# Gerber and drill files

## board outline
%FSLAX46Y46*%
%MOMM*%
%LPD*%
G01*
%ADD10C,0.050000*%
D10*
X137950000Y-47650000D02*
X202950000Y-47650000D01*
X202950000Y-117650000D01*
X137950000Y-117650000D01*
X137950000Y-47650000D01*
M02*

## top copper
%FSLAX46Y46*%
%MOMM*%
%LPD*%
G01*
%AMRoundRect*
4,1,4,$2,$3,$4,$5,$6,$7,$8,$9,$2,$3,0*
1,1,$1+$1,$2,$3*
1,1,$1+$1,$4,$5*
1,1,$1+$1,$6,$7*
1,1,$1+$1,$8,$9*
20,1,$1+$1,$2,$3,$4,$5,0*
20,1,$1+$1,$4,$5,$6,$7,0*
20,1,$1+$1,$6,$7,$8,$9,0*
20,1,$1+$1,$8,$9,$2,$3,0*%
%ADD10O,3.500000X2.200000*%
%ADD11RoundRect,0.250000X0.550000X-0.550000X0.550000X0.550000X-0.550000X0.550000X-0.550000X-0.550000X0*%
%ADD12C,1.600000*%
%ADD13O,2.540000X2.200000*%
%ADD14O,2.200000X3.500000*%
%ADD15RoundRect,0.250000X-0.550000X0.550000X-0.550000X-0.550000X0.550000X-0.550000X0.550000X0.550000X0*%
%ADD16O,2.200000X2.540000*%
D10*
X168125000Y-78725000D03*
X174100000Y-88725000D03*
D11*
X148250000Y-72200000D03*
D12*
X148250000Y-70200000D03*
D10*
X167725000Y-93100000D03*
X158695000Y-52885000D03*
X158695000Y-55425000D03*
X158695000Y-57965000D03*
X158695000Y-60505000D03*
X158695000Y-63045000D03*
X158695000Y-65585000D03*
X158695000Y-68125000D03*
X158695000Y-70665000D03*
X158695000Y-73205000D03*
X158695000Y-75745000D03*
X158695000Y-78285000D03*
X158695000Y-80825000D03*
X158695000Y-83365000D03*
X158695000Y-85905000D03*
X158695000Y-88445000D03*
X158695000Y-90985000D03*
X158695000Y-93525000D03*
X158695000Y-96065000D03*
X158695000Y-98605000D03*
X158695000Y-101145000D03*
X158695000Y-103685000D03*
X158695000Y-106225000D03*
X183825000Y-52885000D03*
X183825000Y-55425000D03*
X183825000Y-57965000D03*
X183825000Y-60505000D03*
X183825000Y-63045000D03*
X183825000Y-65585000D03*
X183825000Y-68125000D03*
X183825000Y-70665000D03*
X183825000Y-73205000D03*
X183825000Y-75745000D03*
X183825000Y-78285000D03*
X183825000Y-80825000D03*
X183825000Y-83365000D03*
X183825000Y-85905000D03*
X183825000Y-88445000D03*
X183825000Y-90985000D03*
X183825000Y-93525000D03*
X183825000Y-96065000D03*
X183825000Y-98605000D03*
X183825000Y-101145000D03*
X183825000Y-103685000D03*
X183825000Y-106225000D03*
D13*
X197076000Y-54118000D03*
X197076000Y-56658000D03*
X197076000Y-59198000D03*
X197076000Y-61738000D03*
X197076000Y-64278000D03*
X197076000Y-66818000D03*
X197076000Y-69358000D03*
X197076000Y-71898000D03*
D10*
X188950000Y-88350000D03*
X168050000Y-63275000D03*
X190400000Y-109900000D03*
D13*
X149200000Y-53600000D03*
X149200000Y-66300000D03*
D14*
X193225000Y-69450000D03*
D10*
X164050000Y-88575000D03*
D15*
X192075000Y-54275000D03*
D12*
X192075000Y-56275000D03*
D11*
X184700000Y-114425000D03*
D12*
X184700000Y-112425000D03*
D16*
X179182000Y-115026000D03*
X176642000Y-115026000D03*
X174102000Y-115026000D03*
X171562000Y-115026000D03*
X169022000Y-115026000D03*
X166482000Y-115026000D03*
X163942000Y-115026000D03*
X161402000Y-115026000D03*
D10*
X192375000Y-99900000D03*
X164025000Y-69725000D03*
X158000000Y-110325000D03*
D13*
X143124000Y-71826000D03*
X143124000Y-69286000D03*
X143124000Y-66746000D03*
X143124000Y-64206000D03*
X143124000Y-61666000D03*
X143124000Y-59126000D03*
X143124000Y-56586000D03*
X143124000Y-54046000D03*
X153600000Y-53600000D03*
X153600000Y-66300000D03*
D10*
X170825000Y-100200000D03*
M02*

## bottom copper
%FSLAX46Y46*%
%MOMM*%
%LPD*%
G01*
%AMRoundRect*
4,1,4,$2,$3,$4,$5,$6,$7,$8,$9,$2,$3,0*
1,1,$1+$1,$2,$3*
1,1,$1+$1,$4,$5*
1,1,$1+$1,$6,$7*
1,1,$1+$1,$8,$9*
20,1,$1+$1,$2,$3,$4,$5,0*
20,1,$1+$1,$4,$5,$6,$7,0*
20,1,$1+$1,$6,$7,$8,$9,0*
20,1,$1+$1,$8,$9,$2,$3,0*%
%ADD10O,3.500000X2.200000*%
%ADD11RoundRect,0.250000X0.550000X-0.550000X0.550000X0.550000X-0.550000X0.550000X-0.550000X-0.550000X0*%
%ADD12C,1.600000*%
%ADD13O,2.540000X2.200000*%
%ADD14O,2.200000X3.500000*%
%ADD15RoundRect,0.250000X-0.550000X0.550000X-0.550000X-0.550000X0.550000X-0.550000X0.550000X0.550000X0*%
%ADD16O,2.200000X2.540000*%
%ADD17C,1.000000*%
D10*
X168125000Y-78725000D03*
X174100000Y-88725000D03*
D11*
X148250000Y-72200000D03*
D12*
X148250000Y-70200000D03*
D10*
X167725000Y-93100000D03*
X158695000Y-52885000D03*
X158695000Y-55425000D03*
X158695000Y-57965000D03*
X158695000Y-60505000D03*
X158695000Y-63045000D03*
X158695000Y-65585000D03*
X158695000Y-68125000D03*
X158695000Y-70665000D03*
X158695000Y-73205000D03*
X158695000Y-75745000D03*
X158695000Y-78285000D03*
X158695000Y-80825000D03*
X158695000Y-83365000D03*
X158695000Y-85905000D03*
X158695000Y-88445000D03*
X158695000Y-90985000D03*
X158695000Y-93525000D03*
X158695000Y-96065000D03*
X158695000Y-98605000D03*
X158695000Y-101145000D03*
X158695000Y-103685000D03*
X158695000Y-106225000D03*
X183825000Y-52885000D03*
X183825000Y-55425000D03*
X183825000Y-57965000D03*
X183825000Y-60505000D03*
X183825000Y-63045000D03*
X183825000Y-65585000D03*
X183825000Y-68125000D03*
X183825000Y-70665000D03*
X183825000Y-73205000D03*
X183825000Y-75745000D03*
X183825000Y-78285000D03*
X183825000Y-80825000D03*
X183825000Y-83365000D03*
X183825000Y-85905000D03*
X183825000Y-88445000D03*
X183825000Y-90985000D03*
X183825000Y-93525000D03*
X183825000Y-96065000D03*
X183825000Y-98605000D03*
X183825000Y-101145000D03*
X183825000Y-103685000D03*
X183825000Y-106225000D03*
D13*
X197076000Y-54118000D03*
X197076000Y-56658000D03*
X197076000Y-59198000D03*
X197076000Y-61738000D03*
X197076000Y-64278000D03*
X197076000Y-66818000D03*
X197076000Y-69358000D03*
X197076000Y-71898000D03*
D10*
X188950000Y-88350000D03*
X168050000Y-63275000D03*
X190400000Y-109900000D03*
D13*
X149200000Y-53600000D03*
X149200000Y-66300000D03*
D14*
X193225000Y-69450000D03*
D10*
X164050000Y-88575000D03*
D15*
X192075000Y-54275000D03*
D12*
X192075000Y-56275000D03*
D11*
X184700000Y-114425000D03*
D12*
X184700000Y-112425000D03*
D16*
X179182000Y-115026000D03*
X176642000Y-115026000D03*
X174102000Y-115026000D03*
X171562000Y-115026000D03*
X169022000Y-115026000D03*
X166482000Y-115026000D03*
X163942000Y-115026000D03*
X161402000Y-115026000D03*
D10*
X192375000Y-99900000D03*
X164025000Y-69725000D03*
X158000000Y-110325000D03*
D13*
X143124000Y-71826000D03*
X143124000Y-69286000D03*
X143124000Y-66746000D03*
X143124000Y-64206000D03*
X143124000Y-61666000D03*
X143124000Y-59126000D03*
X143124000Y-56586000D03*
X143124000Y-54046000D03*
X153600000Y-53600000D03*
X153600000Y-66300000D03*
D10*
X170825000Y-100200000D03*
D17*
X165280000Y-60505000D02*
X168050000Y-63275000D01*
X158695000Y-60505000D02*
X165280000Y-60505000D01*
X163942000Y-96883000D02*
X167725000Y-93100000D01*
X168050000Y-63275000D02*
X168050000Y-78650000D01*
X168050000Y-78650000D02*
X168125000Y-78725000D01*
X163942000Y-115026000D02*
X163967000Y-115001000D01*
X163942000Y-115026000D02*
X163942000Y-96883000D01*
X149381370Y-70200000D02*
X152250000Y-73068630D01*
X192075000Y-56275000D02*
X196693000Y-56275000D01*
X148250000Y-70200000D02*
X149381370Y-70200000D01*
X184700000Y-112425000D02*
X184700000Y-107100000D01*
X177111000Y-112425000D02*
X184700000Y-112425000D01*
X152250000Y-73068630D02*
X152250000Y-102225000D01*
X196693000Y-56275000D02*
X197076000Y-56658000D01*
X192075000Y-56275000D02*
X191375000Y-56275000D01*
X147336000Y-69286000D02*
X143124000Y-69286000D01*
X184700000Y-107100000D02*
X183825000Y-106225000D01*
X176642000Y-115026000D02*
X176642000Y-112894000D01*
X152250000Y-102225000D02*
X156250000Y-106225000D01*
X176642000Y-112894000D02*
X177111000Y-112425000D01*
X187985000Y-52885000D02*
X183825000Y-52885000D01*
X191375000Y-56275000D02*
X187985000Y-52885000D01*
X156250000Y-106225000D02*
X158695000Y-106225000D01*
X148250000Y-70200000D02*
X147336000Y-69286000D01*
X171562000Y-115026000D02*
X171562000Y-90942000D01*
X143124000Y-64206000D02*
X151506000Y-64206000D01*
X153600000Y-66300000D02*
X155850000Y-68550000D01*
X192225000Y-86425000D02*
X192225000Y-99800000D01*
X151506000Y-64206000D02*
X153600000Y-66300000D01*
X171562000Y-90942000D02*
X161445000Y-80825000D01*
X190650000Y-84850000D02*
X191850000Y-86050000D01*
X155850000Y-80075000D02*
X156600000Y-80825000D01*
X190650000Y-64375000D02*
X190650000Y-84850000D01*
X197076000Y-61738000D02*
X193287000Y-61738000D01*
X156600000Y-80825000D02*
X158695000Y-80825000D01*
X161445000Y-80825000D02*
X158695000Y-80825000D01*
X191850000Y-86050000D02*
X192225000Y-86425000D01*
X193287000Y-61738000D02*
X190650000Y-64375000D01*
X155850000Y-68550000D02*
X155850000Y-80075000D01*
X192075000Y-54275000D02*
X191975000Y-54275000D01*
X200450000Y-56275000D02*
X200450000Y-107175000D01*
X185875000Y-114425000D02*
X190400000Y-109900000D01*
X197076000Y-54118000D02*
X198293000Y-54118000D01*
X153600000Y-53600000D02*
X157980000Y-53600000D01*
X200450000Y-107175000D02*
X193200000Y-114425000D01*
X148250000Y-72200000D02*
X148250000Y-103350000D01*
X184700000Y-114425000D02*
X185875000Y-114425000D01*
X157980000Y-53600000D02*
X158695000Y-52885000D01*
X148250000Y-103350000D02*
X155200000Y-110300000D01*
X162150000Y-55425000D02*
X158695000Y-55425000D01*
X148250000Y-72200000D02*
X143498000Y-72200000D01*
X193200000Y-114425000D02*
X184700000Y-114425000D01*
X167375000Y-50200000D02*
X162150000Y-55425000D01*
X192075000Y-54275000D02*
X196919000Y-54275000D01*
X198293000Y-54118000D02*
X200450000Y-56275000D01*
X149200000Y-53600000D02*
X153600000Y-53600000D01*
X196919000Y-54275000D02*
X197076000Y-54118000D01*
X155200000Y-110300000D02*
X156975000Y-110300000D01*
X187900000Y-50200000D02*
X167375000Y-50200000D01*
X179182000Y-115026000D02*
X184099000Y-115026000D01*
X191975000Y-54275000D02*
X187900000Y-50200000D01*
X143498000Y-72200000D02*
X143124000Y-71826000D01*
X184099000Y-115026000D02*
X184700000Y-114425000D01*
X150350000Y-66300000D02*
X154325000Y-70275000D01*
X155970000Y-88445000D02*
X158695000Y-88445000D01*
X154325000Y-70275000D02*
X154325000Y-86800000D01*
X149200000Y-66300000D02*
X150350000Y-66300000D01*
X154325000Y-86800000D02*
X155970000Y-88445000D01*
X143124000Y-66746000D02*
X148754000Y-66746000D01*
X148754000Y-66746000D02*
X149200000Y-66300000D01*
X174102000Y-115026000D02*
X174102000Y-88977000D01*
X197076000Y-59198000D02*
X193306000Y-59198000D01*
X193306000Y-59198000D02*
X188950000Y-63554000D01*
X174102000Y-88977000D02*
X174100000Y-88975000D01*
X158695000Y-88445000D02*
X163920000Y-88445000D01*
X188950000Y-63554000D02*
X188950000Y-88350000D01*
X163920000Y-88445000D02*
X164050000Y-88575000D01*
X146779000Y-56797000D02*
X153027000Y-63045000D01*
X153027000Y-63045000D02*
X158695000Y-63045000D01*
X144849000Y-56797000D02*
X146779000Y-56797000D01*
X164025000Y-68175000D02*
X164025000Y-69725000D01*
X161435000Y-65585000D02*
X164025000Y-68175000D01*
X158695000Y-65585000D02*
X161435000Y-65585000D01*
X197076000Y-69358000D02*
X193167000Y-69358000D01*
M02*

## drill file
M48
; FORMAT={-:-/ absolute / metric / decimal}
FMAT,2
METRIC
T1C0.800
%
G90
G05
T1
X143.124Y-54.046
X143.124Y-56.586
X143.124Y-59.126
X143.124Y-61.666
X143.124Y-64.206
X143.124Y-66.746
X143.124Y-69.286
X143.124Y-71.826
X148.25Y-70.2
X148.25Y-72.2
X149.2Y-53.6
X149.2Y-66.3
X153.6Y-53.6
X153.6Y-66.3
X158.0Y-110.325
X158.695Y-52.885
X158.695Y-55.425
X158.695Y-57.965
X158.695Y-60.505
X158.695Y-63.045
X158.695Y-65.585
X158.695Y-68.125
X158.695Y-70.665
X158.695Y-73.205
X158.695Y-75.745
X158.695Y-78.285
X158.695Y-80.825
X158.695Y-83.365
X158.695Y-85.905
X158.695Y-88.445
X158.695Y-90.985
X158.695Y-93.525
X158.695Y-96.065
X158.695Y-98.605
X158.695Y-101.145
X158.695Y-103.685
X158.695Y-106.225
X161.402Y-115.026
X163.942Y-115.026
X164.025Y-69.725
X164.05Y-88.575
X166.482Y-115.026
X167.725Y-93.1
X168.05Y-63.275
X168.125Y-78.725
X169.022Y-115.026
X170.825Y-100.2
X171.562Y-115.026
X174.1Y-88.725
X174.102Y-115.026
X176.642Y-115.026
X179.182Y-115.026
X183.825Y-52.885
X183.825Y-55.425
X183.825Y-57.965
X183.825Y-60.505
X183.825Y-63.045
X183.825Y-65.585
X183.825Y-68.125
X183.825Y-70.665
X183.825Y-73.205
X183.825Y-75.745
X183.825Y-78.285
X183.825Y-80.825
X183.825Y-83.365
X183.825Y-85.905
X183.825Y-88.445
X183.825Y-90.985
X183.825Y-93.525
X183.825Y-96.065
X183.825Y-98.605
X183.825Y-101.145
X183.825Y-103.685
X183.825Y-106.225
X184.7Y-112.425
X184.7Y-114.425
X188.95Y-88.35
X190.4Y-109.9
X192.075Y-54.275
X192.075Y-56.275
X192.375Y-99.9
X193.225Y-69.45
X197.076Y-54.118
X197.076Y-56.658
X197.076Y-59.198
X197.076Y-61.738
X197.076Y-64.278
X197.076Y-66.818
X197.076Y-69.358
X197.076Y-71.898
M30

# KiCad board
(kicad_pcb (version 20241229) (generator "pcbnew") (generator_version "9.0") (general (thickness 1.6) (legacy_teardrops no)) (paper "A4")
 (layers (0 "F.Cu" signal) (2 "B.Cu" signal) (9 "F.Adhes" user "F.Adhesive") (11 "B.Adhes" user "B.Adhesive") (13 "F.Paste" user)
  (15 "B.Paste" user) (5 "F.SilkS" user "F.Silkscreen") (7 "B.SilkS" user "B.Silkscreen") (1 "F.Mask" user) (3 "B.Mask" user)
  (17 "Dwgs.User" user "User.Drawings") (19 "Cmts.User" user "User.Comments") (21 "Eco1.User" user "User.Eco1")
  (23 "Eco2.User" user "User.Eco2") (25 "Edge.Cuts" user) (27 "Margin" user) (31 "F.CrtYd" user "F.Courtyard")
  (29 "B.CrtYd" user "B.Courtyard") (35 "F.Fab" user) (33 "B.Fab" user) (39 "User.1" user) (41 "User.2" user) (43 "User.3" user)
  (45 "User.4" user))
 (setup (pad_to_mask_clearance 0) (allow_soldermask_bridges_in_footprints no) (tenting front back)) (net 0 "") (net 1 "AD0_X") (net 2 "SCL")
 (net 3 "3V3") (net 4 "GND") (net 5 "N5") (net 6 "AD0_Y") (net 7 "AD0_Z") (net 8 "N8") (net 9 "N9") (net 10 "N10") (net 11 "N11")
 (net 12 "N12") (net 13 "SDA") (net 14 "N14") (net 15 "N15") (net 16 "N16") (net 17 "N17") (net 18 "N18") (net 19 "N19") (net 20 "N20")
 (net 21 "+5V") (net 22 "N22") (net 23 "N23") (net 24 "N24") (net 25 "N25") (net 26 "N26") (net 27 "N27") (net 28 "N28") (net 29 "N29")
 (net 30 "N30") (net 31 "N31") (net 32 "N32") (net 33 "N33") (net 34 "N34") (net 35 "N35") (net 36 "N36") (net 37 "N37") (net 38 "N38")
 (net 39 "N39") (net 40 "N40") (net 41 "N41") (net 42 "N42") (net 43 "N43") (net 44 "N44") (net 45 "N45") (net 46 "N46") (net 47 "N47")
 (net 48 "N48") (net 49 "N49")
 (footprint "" (layer "F.Cu") (at 168.125 78.725)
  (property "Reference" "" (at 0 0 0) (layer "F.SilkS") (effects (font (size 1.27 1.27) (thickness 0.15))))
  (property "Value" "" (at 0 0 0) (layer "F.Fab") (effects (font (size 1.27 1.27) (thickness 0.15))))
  (pad "4" thru_hole oval (at 0 0) (size 3.5 2.2) (drill 0.8) (layers "*.Cu" "*.Mask") (remove_unused_layers no) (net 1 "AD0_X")))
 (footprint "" (layer "F.Cu") (at 174.1 88.725)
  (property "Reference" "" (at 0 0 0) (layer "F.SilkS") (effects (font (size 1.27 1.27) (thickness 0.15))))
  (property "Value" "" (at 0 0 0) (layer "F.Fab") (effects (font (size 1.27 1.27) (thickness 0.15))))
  (pad "SCL" thru_hole oval (at 0 0) (size 3.5 2.2) (drill 0.8) (layers "*.Cu" "*.Mask") (remove_unused_layers no) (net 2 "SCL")))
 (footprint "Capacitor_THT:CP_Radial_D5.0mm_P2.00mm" (layer "F.Cu") (at 148.25 72.2 90)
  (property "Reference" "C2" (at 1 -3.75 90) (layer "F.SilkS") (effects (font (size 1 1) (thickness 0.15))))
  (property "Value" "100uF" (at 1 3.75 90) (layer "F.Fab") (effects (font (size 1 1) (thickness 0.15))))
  (pad "1" thru_hole roundrect (at 0 0 90) (size 1.6 1.6) (drill 0.8) (layers "*.Cu" "*.Mask") (remove_unused_layers no)
   (roundrect_rratio 0.15625) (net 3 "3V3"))
  (pad "2" thru_hole circle (at 2 0 90) (size 1.6 1.6) (drill 0.8) (layers "*.Cu" "*.Mask") (remove_unused_layers no) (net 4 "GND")))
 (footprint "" (layer "F.Cu") (at 167.725 93.1)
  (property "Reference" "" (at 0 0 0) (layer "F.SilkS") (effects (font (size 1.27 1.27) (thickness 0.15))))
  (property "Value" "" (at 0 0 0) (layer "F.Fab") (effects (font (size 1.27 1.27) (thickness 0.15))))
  (pad "4" thru_hole oval (at 0 0) (size 3.5 2.2) (drill 0.8) (layers "*.Cu" "*.Mask") (remove_unused_layers no) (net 1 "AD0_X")))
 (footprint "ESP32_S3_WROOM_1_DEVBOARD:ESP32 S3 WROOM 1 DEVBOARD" (layer "F.Cu") (at 156.325 51.225)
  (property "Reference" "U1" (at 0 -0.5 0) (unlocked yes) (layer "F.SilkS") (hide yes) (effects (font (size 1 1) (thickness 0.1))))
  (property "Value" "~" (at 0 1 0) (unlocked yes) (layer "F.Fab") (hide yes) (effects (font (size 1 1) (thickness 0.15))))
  (pad "1" thru_hole oval (at 2.37 1.66) (size 3.5 2.2) (drill 0.8) (layers "*.Cu" "*.Mask") (remove_unused_layers no) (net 3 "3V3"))
  (pad "2" thru_hole oval (at 2.37 4.2) (size 3.5 2.2) (drill 0.8) (layers "*.Cu" "*.Mask") (remove_unused_layers no) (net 3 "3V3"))
  (pad "3" thru_hole oval (at 2.37 6.74) (size 3.5 2.2) (drill 0.8) (layers "*.Cu" "*.Mask") (remove_unused_layers no) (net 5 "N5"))
  (pad "4" thru_hole oval (at 2.37 9.28) (size 3.5 2.2) (drill 0.8) (layers "*.Cu" "*.Mask") (remove_unused_layers no) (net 1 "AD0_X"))
  (pad "5" thru_hole oval (at 2.37 11.82) (size 3.5 2.2) (drill 0.8) (layers "*.Cu" "*.Mask") (remove_unused_layers no) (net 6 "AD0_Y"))
  (pad "6" thru_hole oval (at 2.37 14.36) (size 3.5 2.2) (drill 0.8) (layers "*.Cu" "*.Mask") (remove_unused_layers no) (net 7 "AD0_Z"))
  (pad "7" thru_hole oval (at 2.37 16.9) (size 3.5 2.2) (drill 0.8) (layers "*.Cu" "*.Mask") (remove_unused_layers no) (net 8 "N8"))
  (pad "8" thru_hole oval (at 2.37 19.44) (size 3.5 2.2) (drill 0.8) (layers "*.Cu" "*.Mask") (remove_unused_layers no) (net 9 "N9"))
  (pad "9" thru_hole oval (at 2.37 21.98) (size 3.5 2.2) (drill 0.8) (layers "*.Cu" "*.Mask") (remove_unused_layers no) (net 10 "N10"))
  (pad "10" thru_hole oval (at 2.37 24.52) (size 3.5 2.2) (drill 0.8) (layers "*.Cu" "*.Mask") (remove_unused_layers no) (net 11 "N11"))
  (pad "11" thru_hole oval (at 2.37 27.06) (size 3.5 2.2) (drill 0.8) (layers "*.Cu" "*.Mask") (remove_unused_layers no) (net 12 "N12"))
  (pad "12" thru_hole oval (at 2.37 29.6) (size 3.5 2.2) (drill 0.8) (layers "*.Cu" "*.Mask") (remove_unused_layers no) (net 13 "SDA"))
  (pad "13" thru_hole oval (at 2.37 32.14) (size 3.5 2.2) (drill 0.8) (layers "*.Cu" "*.Mask") (remove_unused_layers no) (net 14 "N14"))
  (pad "14" thru_hole oval (at 2.37 34.68) (size 3.5 2.2) (drill 0.8) (layers "*.Cu" "*.Mask") (remove_unused_layers no) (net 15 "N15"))
  (pad "15" thru_hole oval (at 2.37 37.22) (size 3.5 2.2) (drill 0.8) (layers "*.Cu" "*.Mask") (remove_unused_layers no) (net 2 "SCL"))
  (pad "16" thru_hole oval (at 2.37 39.76) (size 3.5 2.2) (drill 0.8) (layers "*.Cu" "*.Mask") (remove_unused_layers no) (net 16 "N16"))
  (pad "17" thru_hole oval (at 2.37 42.3) (size 3.5 2.2) (drill 0.8) (layers "*.Cu" "*.Mask") (remove_unused_layers no) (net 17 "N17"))
  (pad "18" thru_hole oval (at 2.37 44.84) (size 3.5 2.2) (drill 0.8) (layers "*.Cu" "*.Mask") (remove_unused_layers no) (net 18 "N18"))
  (pad "19" thru_hole oval (at 2.37 47.38) (size 3.5 2.2) (drill 0.8) (layers "*.Cu" "*.Mask") (remove_unused_layers no) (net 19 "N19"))
  (pad "20" thru_hole oval (at 2.37 49.92) (size 3.5 2.2) (drill 0.8) (layers "*.Cu" "*.Mask") (remove_unused_layers no) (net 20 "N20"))
  (pad "21" thru_hole oval (at 2.37 52.46) (size 3.5 2.2) (drill 0.8) (layers "*.Cu" "*.Mask") (remove_unused_layers no) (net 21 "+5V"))
  (pad "22" thru_hole oval (at 2.37 55) (size 3.5 2.2) (drill 0.8) (layers "*.Cu" "*.Mask") (remove_unused_layers no) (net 4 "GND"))
  (pad "23" thru_hole oval (at 27.5 1.66) (size 3.5 2.2) (drill 0.8) (layers "*.Cu" "*.Mask") (remove_unused_layers no) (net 4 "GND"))
  (pad "24" thru_hole oval (at 27.5 4.2) (size 3.5 2.2) (drill 0.8) (layers "*.Cu" "*.Mask") (remove_unused_layers no) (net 4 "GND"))
  (pad "25" thru_hole oval (at 27.5 6.74) (size 3.5 2.2) (drill 0.8) (layers "*.Cu" "*.Mask") (remove_unused_layers no) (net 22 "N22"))
  (pad "26" thru_hole oval (at 27.5 9.28) (size 3.5 2.2) (drill 0.8) (layers "*.Cu" "*.Mask") (remove_unused_layers no) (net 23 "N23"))
  (pad "27" thru_hole oval (at 27.5 11.82) (size 3.5 2.2) (drill 0.8) (layers "*.Cu" "*.Mask") (remove_unused_layers no) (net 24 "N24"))
  (pad "28" thru_hole oval (at 27.5 14.36) (size 3.5 2.2) (drill 0.8) (layers "*.Cu" "*.Mask") (remove_unused_layers no) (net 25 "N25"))
  (pad "29" thru_hole oval (at 27.5 16.9) (size 3.5 2.2) (drill 0.8) (layers "*.Cu" "*.Mask") (remove_unused_layers no) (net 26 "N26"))
  (pad "30" thru_hole oval (at 27.5 19.44) (size 3.5 2.2) (drill 0.8) (layers "*.Cu" "*.Mask") (remove_unused_layers no) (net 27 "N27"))
  (pad "31" thru_hole oval (at 27.5 21.98) (size 3.5 2.2) (drill 0.8) (layers "*.Cu" "*.Mask") (remove_unused_layers no) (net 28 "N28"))
  (pad "32" thru_hole oval (at 27.5 24.52) (size 3.5 2.2) (drill 0.8) (layers "*.Cu" "*.Mask") (remove_unused_layers no) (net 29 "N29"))
  (pad "33" thru_hole oval (at 27.5 27.06) (size 3.5 2.2) (drill 0.8) (layers "*.Cu" "*.Mask") (remove_unused_layers no) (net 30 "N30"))
  (pad "34" thru_hole oval (at 27.5 29.6) (size 3.5 2.2) (drill 0.8) (layers "*.Cu" "*.Mask") (remove_unused_layers no) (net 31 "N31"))
  (pad "35" thru_hole oval (at 27.5 32.14) (size 3.5 2.2) (drill 0.8) (layers "*.Cu" "*.Mask") (remove_unused_layers no) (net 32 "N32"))
  (pad "36" thru_hole oval (at 27.5 34.68) (size 3.5 2.2) (drill 0.8) (layers "*.Cu" "*.Mask") (remove_unused_layers no) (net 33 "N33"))
  (pad "37" thru_hole oval (at 27.5 37.22) (size 3.5 2.2) (drill 0.8) (layers "*.Cu" "*.Mask") (remove_unused_layers no) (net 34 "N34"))
  (pad "38" thru_hole oval (at 27.5 39.76) (size 3.5 2.2) (drill 0.8) (layers "*.Cu" "*.Mask") (remove_unused_layers no) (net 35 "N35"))
  (pad "39" thru_hole oval (at 27.5 42.3) (size 3.5 2.2) (drill 0.8) (layers "*.Cu" "*.Mask") (remove_unused_layers no) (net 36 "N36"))
  (pad "40" thru_hole oval (at 27.5 44.84) (size 3.5 2.2) (drill 0.8) (layers "*.Cu" "*.Mask") (remove_unused_layers no) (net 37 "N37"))
  (pad "41" thru_hole oval (at 27.5 47.38) (size 3.5 2.2) (drill 0.8) (layers "*.Cu" "*.Mask") (remove_unused_layers no) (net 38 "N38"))
  (pad "42" thru_hole oval (at 27.5 49.92) (size 3.5 2.2) (drill 0.8) (layers "*.Cu" "*.Mask") (remove_unused_layers no) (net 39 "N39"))
  (pad "43" thru_hole oval (at 27.5 52.46) (size 3.5 2.2) (drill 0.8) (layers "*.Cu" "*.Mask") (remove_unused_layers no) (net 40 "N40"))
  (pad "44" thru_hole oval (at 27.5 55) (size 3.5 2.2) (drill 0.8) (layers "*.Cu" "*.Mask") (remove_unused_layers no) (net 4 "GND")))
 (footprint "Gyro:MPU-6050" (layer "F.Cu") (at 211.3 52.594 -90)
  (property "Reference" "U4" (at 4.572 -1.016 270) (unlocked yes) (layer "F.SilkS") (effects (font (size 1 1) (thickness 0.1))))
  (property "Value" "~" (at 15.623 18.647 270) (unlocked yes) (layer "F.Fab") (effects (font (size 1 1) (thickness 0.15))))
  (pad "1" thru_hole oval (at 1.524 14.224) (size 2.54 2.2) (drill 0.8) (layers "*.Cu" "*.Mask") (remove_unused_layers no) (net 3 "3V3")
   (thermal_bridge_angle 45))
  (pad "2" thru_hole oval (at 4.064 14.224) (size 2.54 2.2) (drill 0.8) (layers "*.Cu" "*.Mask") (remove_unused_layers no) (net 4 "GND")
   (thermal_bridge_angle 45))
  (pad "3" thru_hole oval (at 6.604 14.224) (size 2.54 2.2) (drill 0.8) (layers "*.Cu" "*.Mask") (remove_unused_layers no) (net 2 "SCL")
   (thermal_bridge_angle 45))
  (pad "4" thru_hole oval (at 9.144 14.224) (size 2.54 2.2) (drill 0.8) (layers "*.Cu" "*.Mask") (remove_unused_layers no) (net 13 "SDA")
   (thermal_bridge_angle 45))
  (pad "5" thru_hole oval (at 11.684 14.224) (size 2.54 2.2) (drill 0.8) (layers "*.Cu" "*.Mask") (remove_unused_layers no) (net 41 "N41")
   (thermal_bridge_angle 45))
  (pad "6" thru_hole oval (at 14.224 14.224) (size 2.54 2.2) (drill 0.8) (layers "*.Cu" "*.Mask") (remove_unused_layers no) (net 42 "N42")
   (thermal_bridge_angle 45))
  (pad "7" thru_hole oval (at 16.764 14.224) (size 2.54 2.2) (drill 0.8) (layers "*.Cu" "*.Mask") (remove_unused_layers no) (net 7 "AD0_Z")
   (thermal_bridge_angle 45))
  (pad "8" thru_hole oval (at 19.304 14.224) (size 2.54 2.2) (drill 0.8) (layers "*.Cu" "*.Mask") (remove_unused_layers no) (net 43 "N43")
   (thermal_bridge_angle 45)))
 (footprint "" (layer "F.Cu") (at 188.95 88.35)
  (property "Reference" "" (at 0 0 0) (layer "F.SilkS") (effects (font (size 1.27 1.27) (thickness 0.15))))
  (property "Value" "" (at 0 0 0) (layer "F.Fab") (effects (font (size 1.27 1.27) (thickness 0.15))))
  (pad "SCL" thru_hole oval (at 0 0) (size 3.5 2.2) (drill 0.8) (layers "*.Cu" "*.Mask") (remove_unused_layers no)))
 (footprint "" (layer "F.Cu") (at 168.05 63.275)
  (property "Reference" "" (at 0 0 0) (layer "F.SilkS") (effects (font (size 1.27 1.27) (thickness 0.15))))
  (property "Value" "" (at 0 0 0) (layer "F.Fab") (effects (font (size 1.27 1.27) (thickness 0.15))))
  (pad "4" thru_hole oval (at 0 0) (size 3.5 2.2) (drill 0.8) (layers "*.Cu" "*.Mask") (remove_unused_layers no) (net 1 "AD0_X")))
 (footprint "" (layer "F.Cu") (at 190.4 109.9)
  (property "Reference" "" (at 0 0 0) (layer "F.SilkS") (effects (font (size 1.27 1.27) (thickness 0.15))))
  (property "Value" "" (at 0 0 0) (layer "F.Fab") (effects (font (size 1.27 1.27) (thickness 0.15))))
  (pad "1" thru_hole oval (at 0 0) (size 3.5 2.2) (drill 0.8) (layers "*.Cu" "*.Mask") (remove_unused_layers no) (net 3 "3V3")))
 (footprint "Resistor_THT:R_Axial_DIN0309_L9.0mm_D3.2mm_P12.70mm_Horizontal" (layer "F.Cu") (at 149.2 53.6 -90)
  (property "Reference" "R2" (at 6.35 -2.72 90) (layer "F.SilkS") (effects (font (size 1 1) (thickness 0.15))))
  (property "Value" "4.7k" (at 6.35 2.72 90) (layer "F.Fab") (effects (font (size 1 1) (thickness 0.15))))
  (pad "1" thru_hole oval (at 0 0) (size 2.54 2.2) (drill 0.8) (layers "*.Cu" "*.Mask") (remove_unused_layers no) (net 3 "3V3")
   (thermal_bridge_angle 45))
  (pad "2" thru_hole oval (at 12.7 0) (size 2.54 2.2) (drill 0.8) (layers "*.Cu" "*.Mask") (remove_unused_layers no) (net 2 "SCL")
   (thermal_bridge_angle 45)))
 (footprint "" (layer "F.Cu") (at 193.225 69.45 90)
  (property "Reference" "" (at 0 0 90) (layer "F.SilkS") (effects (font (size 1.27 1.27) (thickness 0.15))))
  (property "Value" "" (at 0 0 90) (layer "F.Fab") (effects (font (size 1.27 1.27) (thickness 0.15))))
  (pad "6" thru_hole oval (at 0 0 90) (size 3.5 2.2) (drill 0.8) (layers "*.Cu" "*.Mask") (remove_unused_layers no) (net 7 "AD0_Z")))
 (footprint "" (layer "F.Cu") (at 164.05 88.575)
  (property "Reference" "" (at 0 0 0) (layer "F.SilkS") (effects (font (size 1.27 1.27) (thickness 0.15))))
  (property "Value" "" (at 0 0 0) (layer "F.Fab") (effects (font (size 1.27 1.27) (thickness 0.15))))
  (pad "SCL" thru_hole oval (at 0 0) (size 3.5 2.2) (drill 0.8) (layers "*.Cu" "*.Mask") (remove_unused_layers no) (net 2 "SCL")))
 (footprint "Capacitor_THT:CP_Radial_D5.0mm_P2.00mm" (layer "F.Cu") (at 192.075 54.275 -90)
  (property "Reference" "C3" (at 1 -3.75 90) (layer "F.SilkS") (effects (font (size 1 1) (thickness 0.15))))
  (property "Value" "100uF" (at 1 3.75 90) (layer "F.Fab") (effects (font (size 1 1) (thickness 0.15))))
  (pad "1" thru_hole roundrect (at 0 0 270) (size 1.6 1.6) (drill 0.8) (layers "*.Cu" "*.Mask") (remove_unused_layers no)
   (roundrect_rratio 0.15625) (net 3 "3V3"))
  (pad "2" thru_hole circle (at 2 0 270) (size 1.6 1.6) (drill 0.8) (layers "*.Cu" "*.Mask") (remove_unused_layers no) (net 4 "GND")))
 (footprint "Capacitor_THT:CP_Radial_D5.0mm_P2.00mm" (layer "F.Cu") (at 184.7 114.425 90)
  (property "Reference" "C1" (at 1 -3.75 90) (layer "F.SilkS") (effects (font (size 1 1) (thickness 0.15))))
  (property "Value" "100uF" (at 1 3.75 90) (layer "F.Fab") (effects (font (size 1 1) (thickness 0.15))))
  (pad "1" thru_hole roundrect (at 0 0 90) (size 1.6 1.6) (drill 0.8) (layers "*.Cu" "*.Mask") (remove_unused_layers no)
   (roundrect_rratio 0.15625) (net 3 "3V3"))
  (pad "2" thru_hole circle (at 2 0 90) (size 1.6 1.6) (drill 0.8) (layers "*.Cu" "*.Mask") (remove_unused_layers no) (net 4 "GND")))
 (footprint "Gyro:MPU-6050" (layer "F.Cu") (at 180.706 129.25 180)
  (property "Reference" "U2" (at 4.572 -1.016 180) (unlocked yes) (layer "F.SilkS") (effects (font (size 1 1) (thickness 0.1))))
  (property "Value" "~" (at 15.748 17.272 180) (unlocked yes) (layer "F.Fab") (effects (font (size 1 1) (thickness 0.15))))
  (pad "1" thru_hole oval (at 1.524 14.224 270) (size 2.54 2.2) (drill 0.8) (layers "*.Cu" "*.Mask") (remove_unused_layers no) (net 3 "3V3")
   (thermal_bridge_angle 45))
  (pad "2" thru_hole oval (at 4.064 14.224 270) (size 2.54 2.2) (drill 0.8) (layers "*.Cu" "*.Mask") (remove_unused_layers no) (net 4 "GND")
   (thermal_bridge_angle 45))
  (pad "3" thru_hole oval (at 6.604 14.224 270) (size 2.54 2.2) (drill 0.8) (layers "*.Cu" "*.Mask") (remove_unused_layers no) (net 2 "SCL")
   (thermal_bridge_angle 45))
  (pad "4" thru_hole oval (at 9.144 14.224 270) (size 2.54 2.2) (drill 0.8) (layers "*.Cu" "*.Mask") (remove_unused_layers no)
   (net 13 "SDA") (thermal_bridge_angle 45))
  (pad "5" thru_hole oval (at 11.684 14.224 270) (size 2.54 2.2) (drill 0.8) (layers "*.Cu" "*.Mask") (remove_unused_layers no)
   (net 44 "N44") (thermal_bridge_angle 45))
  (pad "6" thru_hole oval (at 14.224 14.224 270) (size 2.54 2.2) (drill 0.8) (layers "*.Cu" "*.Mask") (remove_unused_layers no)
   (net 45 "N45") (thermal_bridge_angle 45))
  (pad "7" thru_hole oval (at 16.764 14.224 270) (size 2.54 2.2) (drill 0.8) (layers "*.Cu" "*.Mask") (remove_unused_layers no)
   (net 1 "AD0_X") (thermal_bridge_angle 45))
  (pad "8" thru_hole oval (at 19.304 14.224 270) (size 2.54 2.2) (drill 0.8) (layers "*.Cu" "*.Mask") (remove_unused_layers no)
   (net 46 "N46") (thermal_bridge_angle 45)))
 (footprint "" (layer "F.Cu") (at 192.375 99.9)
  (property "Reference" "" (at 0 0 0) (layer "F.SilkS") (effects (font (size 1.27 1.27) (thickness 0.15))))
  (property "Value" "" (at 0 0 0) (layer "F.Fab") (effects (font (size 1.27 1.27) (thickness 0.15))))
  (pad "12" thru_hole oval (at 0 0) (size 3.5 2.2) (drill 0.8) (layers "*.Cu" "*.Mask") (remove_unused_layers no) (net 13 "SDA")))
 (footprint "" (layer "F.Cu") (at 164.025 69.725)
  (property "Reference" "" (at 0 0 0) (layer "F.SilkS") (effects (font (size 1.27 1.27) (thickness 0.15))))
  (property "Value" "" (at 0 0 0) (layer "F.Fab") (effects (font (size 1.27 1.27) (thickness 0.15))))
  (pad "6" thru_hole oval (at 0 0) (size 3.5 2.2) (drill 0.8) (layers "*.Cu" "*.Mask") (remove_unused_layers no) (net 7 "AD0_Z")))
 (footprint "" (layer "F.Cu") (at 158 110.325)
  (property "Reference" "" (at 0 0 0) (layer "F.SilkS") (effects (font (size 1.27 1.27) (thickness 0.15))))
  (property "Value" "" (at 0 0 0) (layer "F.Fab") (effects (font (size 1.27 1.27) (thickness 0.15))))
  (pad "1" thru_hole oval (at 0 0) (size 3.5 2.2) (drill 0.8) (layers "*.Cu" "*.Mask") (remove_unused_layers no) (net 3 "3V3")))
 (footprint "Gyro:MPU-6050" (layer "F.Cu") (at 128.9 73.35 90)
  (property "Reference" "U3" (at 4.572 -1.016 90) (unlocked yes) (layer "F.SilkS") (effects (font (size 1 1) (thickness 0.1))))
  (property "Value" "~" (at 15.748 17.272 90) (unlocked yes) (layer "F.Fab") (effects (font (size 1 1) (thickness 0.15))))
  (pad "1" thru_hole oval (at 1.524 14.224 180) (size 2.54 2.2) (drill 0.8) (layers "*.Cu" "*.Mask") (remove_unused_layers no) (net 3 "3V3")
   (thermal_bridge_angle 45))
  (pad "2" thru_hole oval (at 4.064 14.224 180) (size 2.54 2.2) (drill 0.8) (layers "*.Cu" "*.Mask") (remove_unused_layers no) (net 4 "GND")
   (thermal_bridge_angle 45))
  (pad "3" thru_hole oval (at 6.604 14.224 180) (size 2.54 2.2) (drill 0.8) (layers "*.Cu" "*.Mask") (remove_unused_layers no) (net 2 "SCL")
   (thermal_bridge_angle 45))
  (pad "4" thru_hole oval (at 9.144 14.224 180) (size 2.54 2.2) (drill 0.8) (layers "*.Cu" "*.Mask") (remove_unused_layers no)
   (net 13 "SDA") (thermal_bridge_angle 45))
  (pad "5" thru_hole oval (at 11.684 14.224 180) (size 2.54 2.2) (drill 0.8) (layers "*.Cu" "*.Mask") (remove_unused_layers no)
   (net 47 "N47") (thermal_bridge_angle 45))
  (pad "6" thru_hole oval (at 14.224 14.224 180) (size 2.54 2.2) (drill 0.8) (layers "*.Cu" "*.Mask") (remove_unused_layers no)
   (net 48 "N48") (thermal_bridge_angle 45))
  (pad "7" thru_hole oval (at 16.764 14.224 180) (size 2.54 2.2) (drill 0.8) (layers "*.Cu" "*.Mask") (remove_unused_layers no)
   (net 6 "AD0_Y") (thermal_bridge_angle 45))
  (pad "8" thru_hole oval (at 19.304 14.224 180) (size 2.54 2.2) (drill 0.8) (layers "*.Cu" "*.Mask") (remove_unused_layers no)
   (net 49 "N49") (thermal_bridge_angle 45)))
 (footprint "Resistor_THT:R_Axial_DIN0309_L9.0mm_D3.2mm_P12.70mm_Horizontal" (layer "F.Cu") (at 153.6 53.6 -90)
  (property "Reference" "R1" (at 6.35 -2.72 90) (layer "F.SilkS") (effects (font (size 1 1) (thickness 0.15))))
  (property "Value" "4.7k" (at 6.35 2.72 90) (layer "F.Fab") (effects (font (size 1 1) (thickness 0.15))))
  (pad "1" thru_hole oval (at 0 0) (size 2.54 2.2) (drill 0.8) (layers "*.Cu" "*.Mask") (remove_unused_layers no) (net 3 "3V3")
   (thermal_bridge_angle 45))
  (pad "2" thru_hole oval (at 12.7 0) (size 2.54 2.2) (drill 0.8) (layers "*.Cu" "*.Mask") (remove_unused_layers no) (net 13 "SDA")
   (thermal_bridge_angle 45)))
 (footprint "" (layer "F.Cu") (at 170.825 100.2)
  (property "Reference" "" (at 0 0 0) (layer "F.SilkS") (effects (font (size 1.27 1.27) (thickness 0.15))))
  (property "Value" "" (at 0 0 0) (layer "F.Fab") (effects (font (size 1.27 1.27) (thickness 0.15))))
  (pad "12" thru_hole oval (at 0 0) (size 3.5 2.2) (drill 0.8) (layers "*.Cu" "*.Mask") (remove_unused_layers no) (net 13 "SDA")))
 (gr_rect (start 137.95 47.65) (end 202.95 117.65) (stroke (width 0.05) (type solid)) (fill no) (layer "Edge.Cuts"))
 (segment (start 165.28 60.505) (end 168.05 63.275) (width 1) (layer "B.Cu") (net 1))
 (segment (start 158.695 60.505) (end 165.28 60.505) (width 1) (layer "B.Cu") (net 1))
 (segment (start 163.942 96.883) (end 167.725 93.1) (width 1) (layer "B.Cu") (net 1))
 (segment (start 168.05 63.275) (end 168.05 78.65) (width 1) (layer "B.Cu") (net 1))
 (segment (start 168.05 78.65) (end 168.125 78.725) (width 1) (layer "B.Cu") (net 1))
 (segment (start 163.942 115.026) (end 163.967 115.001) (width 1) (layer "B.Cu") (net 1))
 (segment (start 163.942 115.026) (end 163.942 96.883) (width 1) (layer "B.Cu") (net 1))
 (segment (start 149.38137 70.2) (end 152.25 73.06863) (width 1) (layer "B.Cu") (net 4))
 (segment (start 192.075 56.275) (end 196.693 56.275) (width 1) (layer "B.Cu") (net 4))
 (segment (start 148.25 70.2) (end 149.38137 70.2) (width 1) (layer "B.Cu") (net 4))
 (segment (start 184.7 112.425) (end 184.7 107.1) (width 1) (layer "B.Cu") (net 4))
 (segment (start 177.111 112.425) (end 184.7 112.425) (width 1) (layer "B.Cu") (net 4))
 (segment (start 152.25 73.06863) (end 152.25 102.225) (width 1) (layer "B.Cu") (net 4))
 (segment (start 196.693 56.275) (end 197.076 56.658) (width 1) (layer "B.Cu") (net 4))
 (segment (start 192.075 56.275) (end 191.375 56.275) (width 1) (layer "B.Cu") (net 4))
 (segment (start 147.336 69.286) (end 143.124 69.286) (width 1) (layer "B.Cu") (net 4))
 (segment (start 184.7 107.1) (end 183.825 106.225) (width 1) (layer "B.Cu") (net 4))
 (segment (start 176.642 115.026) (end 176.642 112.894) (width 1) (layer "B.Cu") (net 4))
 (segment (start 152.25 102.225) (end 156.25 106.225) (width 1) (layer "B.Cu") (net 4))
 (segment (start 176.642 112.894) (end 177.111 112.425) (width 1) (layer "B.Cu") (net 4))
 (segment (start 187.985 52.885) (end 183.825 52.885) (width 1) (layer "B.Cu") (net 4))
 (segment (start 191.375 56.275) (end 187.985 52.885) (width 1) (layer "B.Cu") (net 4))
 (segment (start 156.25 106.225) (end 158.695 106.225) (width 1) (layer "B.Cu") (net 4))
 (segment (start 148.25 70.2) (end 147.336 69.286) (width 1) (layer "B.Cu") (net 4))
 (segment (start 171.562 115.026) (end 171.562 90.942) (width 1) (layer "B.Cu") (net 13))
 (segment (start 143.124 64.206) (end 151.506 64.206) (width 1) (layer "B.Cu") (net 13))
 (segment (start 153.6 66.3) (end 155.85 68.55) (width 1) (layer "B.Cu") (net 13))
 (segment (start 192.225 86.425) (end 192.225 99.8) (width 1) (layer "B.Cu") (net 13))
 (segment (start 151.506 64.206) (end 153.6 66.3) (width 1) (layer "B.Cu") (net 13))
 (segment (start 171.562 90.942) (end 161.445 80.825) (width 1) (layer "B.Cu") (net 13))
 (segment (start 190.65 84.85) (end 191.85 86.05) (width 1) (layer "B.Cu") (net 13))
 (segment (start 155.85 80.075) (end 156.6 80.825) (width 1) (layer "B.Cu") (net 13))
 (segment (start 190.65 64.375) (end 190.65 84.85) (width 1) (layer "B.Cu") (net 13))
 (segment (start 197.076 61.738) (end 193.287 61.738) (width 1) (layer "B.Cu") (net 13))
 (segment (start 156.6 80.825) (end 158.695 80.825) (width 1) (layer "B.Cu") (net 13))
 (segment (start 161.445 80.825) (end 158.695 80.825) (width 1) (layer "B.Cu") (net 13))
 (segment (start 191.85 86.05) (end 192.225 86.425) (width 1) (layer "B.Cu") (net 13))
 (segment (start 193.287 61.738) (end 190.65 64.375) (width 1) (layer "B.Cu") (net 13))
 (segment (start 155.85 68.55) (end 155.85 80.075) (width 1) (layer "B.Cu") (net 13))
 (segment (start 192.075 54.275) (end 191.975 54.275) (width 1) (layer "B.Cu") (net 3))
 (segment (start 200.45 56.275) (end 200.45 107.175) (width 1) (layer "B.Cu") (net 3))
 (segment (start 185.875 114.425) (end 190.4 109.9) (width 1) (layer "B.Cu") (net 3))
 (segment (start 197.076 54.118) (end 198.293 54.118) (width 1) (layer "B.Cu") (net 3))
 (segment (start 153.6 53.6) (end 157.98 53.6) (width 1) (layer "B.Cu") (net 3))
 (segment (start 200.45 107.175) (end 193.2 114.425) (width 1) (layer "B.Cu") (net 3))
 (segment (start 148.25 72.2) (end 148.25 103.35) (width 1) (layer "B.Cu") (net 3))
 (segment (start 184.7 114.425) (end 185.875 114.425) (width 1) (layer "B.Cu") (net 3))
 (segment (start 157.98 53.6) (end 158.695 52.885) (width 1) (layer "B.Cu") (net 3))
 (segment (start 148.25 103.35) (end 155.2 110.3) (width 1) (layer "B.Cu") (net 3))
 (segment (start 162.15 55.425) (end 158.695 55.425) (width 1) (layer "B.Cu") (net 3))
 (segment (start 148.25 72.2) (end 143.498 72.2) (width 1) (layer "B.Cu") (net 3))
 (segment (start 193.2 114.425) (end 184.7 114.425) (width 1) (layer "B.Cu") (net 3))
 (segment (start 167.375 50.2) (end 162.15 55.425) (width 1) (layer "B.Cu") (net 3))
 (segment (start 192.075 54.275) (end 196.919 54.275) (width 1) (layer "B.Cu") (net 3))
 (segment (start 198.293 54.118) (end 200.45 56.275) (width 1) (layer "B.Cu") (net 3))
 (segment (start 149.2 53.6) (end 153.6 53.6) (width 1) (layer "B.Cu") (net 3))
 (segment (start 196.919 54.275) (end 197.076 54.118) (width 1) (layer "B.Cu") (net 3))
 (segment (start 155.2 110.3) (end 156.975 110.3) (width 1) (layer "B.Cu") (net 3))
 (segment (start 187.9 50.2) (end 167.375 50.2) (width 1) (layer "B.Cu") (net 3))
 (segment (start 179.182 115.026) (end 184.099 115.026) (width 1) (layer "B.Cu") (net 3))
 (segment (start 191.975 54.275) (end 187.9 50.2) (width 1) (layer "B.Cu") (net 3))
 (segment (start 143.498 72.2) (end 143.124 71.826) (width 1) (layer "B.Cu") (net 3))
 (segment (start 184.099 115.026) (end 184.7 114.425) (width 1) (layer "B.Cu") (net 3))
 (segment (start 150.35 66.3) (end 154.325 70.275) (width 1) (layer "B.Cu") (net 2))
 (segment (start 155.97 88.445) (end 158.695 88.445) (width 1) (layer "B.Cu") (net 2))
 (segment (start 154.325 70.275) (end 154.325 86.8) (width 1) (layer "B.Cu") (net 2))
 (segment (start 149.2 66.3) (end 150.35 66.3) (width 1) (layer "B.Cu") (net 2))
 (segment (start 154.325 86.8) (end 155.97 88.445) (width 1) (layer "B.Cu") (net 2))
 (segment (start 143.124 66.746) (end 148.754 66.746) (width 1) (layer "B.Cu") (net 2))
 (segment (start 148.754 66.746) (end 149.2 66.3) (width 1) (layer "B.Cu") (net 2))
 (segment (start 174.102 115.026) (end 174.102 88.977) (width 1) (layer "B.Cu") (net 2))
 (segment (start 197.076 59.198) (end 193.306 59.198) (width 1) (layer "B.Cu") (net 2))
 (segment (start 193.306 59.198) (end 188.95 63.554) (width 1) (layer "B.Cu") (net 2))
 (segment (start 174.102 88.977) (end 174.1 88.975) (width 1) (layer "B.Cu") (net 2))
 (segment (start 158.695 88.445) (end 163.92 88.445) (width 1) (layer "B.Cu") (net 2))
 (segment (start 188.95 63.554) (end 188.95 88.35) (width 1) (layer "B.Cu") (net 2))
 (segment (start 163.92 88.445) (end 164.05 88.575) (width 1) (layer "B.Cu") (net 2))
 (segment (start 146.779 56.797) (end 153.027 63.045) (width 1) (layer "B.Cu") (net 6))
 (segment (start 153.027 63.045) (end 158.695 63.045) (width 1) (layer "B.Cu") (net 6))
 (segment (start 144.849 56.797) (end 146.779 56.797) (width 1) (layer "B.Cu") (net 6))
 (segment (start 164.025 68.175) (end 164.025 69.725) (width 1) (layer "B.Cu") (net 7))
 (segment (start 161.435 65.585) (end 164.025 68.175) (width 1) (layer "B.Cu") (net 7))
 (segment (start 158.695 65.585) (end 161.435 65.585) (width 1) (layer "B.Cu") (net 7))
 (segment (start 197.076 69.358) (end 193.167 69.358) (width 1) (layer "B.Cu") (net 7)))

